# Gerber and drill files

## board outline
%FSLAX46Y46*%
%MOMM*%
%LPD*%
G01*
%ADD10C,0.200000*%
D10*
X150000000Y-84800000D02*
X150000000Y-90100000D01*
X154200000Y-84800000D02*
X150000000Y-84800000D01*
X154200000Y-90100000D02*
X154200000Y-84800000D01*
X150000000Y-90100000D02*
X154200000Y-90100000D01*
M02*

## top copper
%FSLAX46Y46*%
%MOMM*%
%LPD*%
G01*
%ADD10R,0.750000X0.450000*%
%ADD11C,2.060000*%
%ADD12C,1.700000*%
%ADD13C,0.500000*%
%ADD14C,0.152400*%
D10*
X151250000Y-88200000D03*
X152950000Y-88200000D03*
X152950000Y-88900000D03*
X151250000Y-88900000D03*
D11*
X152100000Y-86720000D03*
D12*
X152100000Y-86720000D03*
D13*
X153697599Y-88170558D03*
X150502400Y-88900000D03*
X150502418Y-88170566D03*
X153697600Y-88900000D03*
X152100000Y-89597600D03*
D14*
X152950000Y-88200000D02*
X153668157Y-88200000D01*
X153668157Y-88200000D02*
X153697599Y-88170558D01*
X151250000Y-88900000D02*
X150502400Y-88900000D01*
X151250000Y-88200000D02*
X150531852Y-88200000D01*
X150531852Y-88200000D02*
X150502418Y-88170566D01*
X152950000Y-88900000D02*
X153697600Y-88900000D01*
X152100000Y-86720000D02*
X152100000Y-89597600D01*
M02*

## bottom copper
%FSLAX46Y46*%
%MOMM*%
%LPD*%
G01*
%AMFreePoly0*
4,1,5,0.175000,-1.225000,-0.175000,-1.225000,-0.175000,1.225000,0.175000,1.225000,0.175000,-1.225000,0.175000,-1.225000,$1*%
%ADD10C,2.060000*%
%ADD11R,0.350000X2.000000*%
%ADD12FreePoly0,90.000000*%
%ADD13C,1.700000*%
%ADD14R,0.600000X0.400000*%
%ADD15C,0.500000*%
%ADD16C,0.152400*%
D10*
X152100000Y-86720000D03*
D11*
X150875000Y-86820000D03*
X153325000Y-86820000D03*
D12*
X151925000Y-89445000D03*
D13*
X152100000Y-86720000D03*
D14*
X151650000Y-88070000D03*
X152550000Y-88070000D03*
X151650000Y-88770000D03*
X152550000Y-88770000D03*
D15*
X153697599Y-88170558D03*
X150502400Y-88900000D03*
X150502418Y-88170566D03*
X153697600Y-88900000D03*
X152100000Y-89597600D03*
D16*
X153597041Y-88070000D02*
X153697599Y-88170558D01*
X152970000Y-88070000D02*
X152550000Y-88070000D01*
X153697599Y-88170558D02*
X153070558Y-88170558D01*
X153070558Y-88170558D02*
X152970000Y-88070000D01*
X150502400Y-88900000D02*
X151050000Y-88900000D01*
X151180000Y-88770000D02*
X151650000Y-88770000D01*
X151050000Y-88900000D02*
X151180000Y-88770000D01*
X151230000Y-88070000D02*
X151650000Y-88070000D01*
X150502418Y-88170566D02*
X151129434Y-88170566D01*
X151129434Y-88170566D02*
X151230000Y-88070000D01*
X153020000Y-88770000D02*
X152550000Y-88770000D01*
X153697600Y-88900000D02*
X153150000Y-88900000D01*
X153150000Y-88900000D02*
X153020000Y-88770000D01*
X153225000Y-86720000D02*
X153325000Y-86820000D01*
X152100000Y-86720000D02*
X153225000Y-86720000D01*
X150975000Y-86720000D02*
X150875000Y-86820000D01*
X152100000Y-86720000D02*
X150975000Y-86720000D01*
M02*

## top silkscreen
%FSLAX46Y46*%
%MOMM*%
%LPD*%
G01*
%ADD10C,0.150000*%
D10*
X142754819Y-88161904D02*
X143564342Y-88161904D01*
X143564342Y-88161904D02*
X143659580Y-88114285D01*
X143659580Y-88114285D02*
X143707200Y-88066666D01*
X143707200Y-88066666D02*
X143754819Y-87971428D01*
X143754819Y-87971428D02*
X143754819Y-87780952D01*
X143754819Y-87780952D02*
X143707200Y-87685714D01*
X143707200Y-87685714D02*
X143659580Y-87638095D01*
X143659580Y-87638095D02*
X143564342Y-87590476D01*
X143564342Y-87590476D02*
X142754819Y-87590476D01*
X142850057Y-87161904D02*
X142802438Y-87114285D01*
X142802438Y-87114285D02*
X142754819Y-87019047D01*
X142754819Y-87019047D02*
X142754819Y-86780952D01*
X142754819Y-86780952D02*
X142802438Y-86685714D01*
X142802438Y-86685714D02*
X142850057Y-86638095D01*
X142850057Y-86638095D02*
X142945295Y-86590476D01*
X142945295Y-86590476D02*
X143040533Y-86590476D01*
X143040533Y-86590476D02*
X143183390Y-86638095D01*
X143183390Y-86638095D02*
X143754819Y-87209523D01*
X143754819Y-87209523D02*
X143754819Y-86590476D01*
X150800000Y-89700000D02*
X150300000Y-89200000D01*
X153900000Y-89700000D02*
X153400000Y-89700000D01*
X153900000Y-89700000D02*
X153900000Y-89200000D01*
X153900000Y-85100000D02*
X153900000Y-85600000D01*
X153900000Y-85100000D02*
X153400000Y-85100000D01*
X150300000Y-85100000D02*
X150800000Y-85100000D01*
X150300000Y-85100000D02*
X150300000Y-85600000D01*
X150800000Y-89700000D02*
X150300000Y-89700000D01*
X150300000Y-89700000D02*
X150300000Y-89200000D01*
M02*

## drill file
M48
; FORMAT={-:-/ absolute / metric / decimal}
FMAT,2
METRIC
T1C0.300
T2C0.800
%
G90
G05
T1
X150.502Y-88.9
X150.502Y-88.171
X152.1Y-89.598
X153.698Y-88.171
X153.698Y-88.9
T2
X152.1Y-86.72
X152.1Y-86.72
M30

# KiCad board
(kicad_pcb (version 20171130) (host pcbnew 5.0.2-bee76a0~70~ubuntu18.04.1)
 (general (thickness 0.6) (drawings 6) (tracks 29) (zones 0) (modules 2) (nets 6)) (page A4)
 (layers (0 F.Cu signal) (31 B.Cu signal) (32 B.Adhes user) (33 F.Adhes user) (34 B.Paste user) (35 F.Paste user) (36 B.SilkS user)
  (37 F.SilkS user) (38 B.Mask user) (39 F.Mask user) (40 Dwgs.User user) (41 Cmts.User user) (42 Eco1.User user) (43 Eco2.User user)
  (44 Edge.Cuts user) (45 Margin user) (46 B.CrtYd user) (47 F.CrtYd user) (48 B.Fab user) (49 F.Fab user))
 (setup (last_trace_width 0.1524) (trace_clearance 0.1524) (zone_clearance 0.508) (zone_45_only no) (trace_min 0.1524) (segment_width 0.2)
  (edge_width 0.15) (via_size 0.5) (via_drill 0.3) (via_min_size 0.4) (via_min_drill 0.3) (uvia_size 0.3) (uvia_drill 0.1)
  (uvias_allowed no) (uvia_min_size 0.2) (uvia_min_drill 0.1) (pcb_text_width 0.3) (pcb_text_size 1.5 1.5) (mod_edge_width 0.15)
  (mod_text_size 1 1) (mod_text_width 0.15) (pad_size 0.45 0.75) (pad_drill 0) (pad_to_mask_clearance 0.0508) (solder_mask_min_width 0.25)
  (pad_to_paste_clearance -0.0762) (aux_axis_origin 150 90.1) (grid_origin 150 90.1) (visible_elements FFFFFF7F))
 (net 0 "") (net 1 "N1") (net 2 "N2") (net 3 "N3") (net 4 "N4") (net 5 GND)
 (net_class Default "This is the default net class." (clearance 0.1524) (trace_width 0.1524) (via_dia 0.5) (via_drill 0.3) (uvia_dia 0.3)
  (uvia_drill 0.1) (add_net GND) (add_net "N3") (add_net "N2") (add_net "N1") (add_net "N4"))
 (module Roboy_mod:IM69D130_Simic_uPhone (layer F.Cu) (at 152.1 87.4 90)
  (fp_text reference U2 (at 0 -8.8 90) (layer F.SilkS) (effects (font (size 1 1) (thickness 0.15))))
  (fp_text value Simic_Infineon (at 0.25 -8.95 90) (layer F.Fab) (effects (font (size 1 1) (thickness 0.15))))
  (fp_line (start -2.3 -1.3) (end -1.8 -1.8) (layer F.SilkS) (width 0.15))
  (fp_line (start -2.3 1.8) (end -2.3 1.3) (layer F.SilkS) (width 0.15))
  (fp_line (start -2.3 1.8) (end -1.8 1.8) (layer F.SilkS) (width 0.15))
  (fp_line (start 2.3 1.8) (end 1.8 1.8) (layer F.SilkS) (width 0.15))
  (fp_line (start 2.3 1.8) (end 2.3 1.3) (layer F.SilkS) (width 0.15))
  (fp_line (start 2.3 -1.8) (end 2.3 -1.3) (layer F.SilkS) (width 0.15))
  (fp_line (start 2.3 -1.8) (end 1.8 -1.8) (layer F.SilkS) (width 0.15))
  (fp_line (start -2.3 -1.3) (end -2.3 -1.8) (layer F.SilkS) (width 0.15))
  (fp_line (start -2.3 -1.8) (end -1.8 -1.8) (layer F.SilkS) (width 0.15))
  (pad 2 smd rect (at -0.8 -0.85 90) (size 0.45 0.75) (layers F.Cu F.Paste F.Mask) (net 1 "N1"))
  (pad 4 smd rect (at -0.8 0.85 90) (size 0.45 0.75) (layers F.Cu F.Paste F.Mask) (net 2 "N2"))
  (pad 3 smd rect (at -1.5 0.85 90) (size 0.45 0.75) (layers F.Cu F.Paste F.Mask) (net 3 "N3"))
  (pad 1 smd rect (at -1.5 -0.85 90) (size 0.45 0.75) (layers F.Cu F.Paste F.Mask) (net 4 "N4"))
  (pad 5 thru_hole circle (at 0.68 0 90) (size 2.06 2.06) (drill 0.8) (layers F.Cu) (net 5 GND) (zone_connect 0)))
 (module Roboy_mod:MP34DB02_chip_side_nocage (layer B.Cu) (at 152.1 87.72 90)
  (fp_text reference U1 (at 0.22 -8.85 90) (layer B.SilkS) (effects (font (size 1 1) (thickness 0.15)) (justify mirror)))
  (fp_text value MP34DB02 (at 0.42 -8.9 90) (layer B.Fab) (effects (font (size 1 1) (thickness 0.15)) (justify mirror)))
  (pad 5 smd rect (at 0.9 -1.225 90) (size 2 0.35) (layers B.Cu B.Paste B.Mask) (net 5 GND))
  (pad 5 smd rect (at 0.9 1.225 90) (size 2 0.35) (layers B.Cu B.Paste B.Mask) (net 5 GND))
  (pad 5 smd custom (at -1.725 -0.175 90) (size 0.35 2.45) (layers B.Cu B.Paste B.Mask) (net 5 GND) (zone_connect 0)
   (options (clearance outline) (anchor rect)) (primitives))
  (pad 5 thru_hole circle (at 1 0 90) (size 1.7 1.7) (drill 0.8) (layers B.Cu) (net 5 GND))
  (pad 3 smd rect (at -0.35 -0.45 90) (size 0.4 0.6) (layers B.Cu B.Paste B.Mask) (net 1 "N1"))
  (pad 2 smd rect (at -0.35 0.45 90) (size 0.4 0.6) (layers B.Cu B.Paste B.Mask) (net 2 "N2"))
  (pad 4 smd rect (at -1.05 -0.45 90) (size 0.4 0.6) (layers B.Cu B.Paste B.Mask) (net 4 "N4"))
  (pad 1 smd rect (at -1.05 0.45 90) (size 0.4 0.6) (layers B.Cu B.Paste B.Mask) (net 3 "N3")))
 (gr_line (start 150 84.8) (end 150 90.1) (layer Edge.Cuts) (width 0.2))
 (gr_line (start 154.2 84.8) (end 150 84.8) (layer Edge.Cuts) (width 0.2))
 (gr_line (start 154.2 90.1) (end 154.2 84.8) (layer Edge.Cuts) (width 0.2))
 (gr_line (start 150 90.1) (end 154.2 90.1) (layer Edge.Cuts) (width 0.2))
 (via (at 153.697599 88.170558) (size 0.5) (drill 0.3) (layers F.Cu B.Cu) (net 2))
 (segment (start 152.95 88.2) (end 153.668157 88.2) (width 0.1524) (layer F.Cu) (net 2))
 (segment (start 153.668157 88.2) (end 153.697599 88.170558) (width 0.1524) (layer F.Cu) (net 2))
 (segment (start 153.597041 88.07) (end 153.697599 88.170558) (width 0.1524) (layer B.Cu) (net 2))
 (segment (start 152.97 88.07) (end 152.55 88.07) (width 0.1524) (layer B.Cu) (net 2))
 (segment (start 153.697599 88.170558) (end 153.070558 88.170558) (width 0.1524) (layer B.Cu) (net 2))
 (segment (start 153.070558 88.170558) (end 152.97 88.07) (width 0.1524) (layer B.Cu) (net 2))
 (via (at 150.5024 88.9) (size 0.5) (drill 0.3) (layers F.Cu B.Cu) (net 4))
 (segment (start 151.25 88.9) (end 150.5024 88.9) (width 0.1524) (layer F.Cu) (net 4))
 (segment (start 150.5024 88.9) (end 151.05 88.9) (width 0.1524) (layer B.Cu) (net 4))
 (segment (start 151.18 88.77) (end 151.65 88.77) (width 0.1524) (layer B.Cu) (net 4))
 (segment (start 151.05 88.9) (end 151.18 88.77) (width 0.1524) (layer B.Cu) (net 4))
 (via (at 150.502418 88.170566) (size 0.5) (drill 0.3) (layers F.Cu B.Cu) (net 1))
 (segment (start 151.25 88.2) (end 150.531852 88.2) (width 0.1524) (layer F.Cu) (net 1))
 (segment (start 150.531852 88.2) (end 150.502418 88.170566) (width 0.1524) (layer F.Cu) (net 1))
 (segment (start 151.23 88.07) (end 151.65 88.07) (width 0.1524) (layer B.Cu) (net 1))
 (segment (start 150.502418 88.170566) (end 151.129434 88.170566) (width 0.1524) (layer B.Cu) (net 1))
 (segment (start 151.129434 88.170566) (end 151.23 88.07) (width 0.1524) (layer B.Cu) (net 1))
 (via (at 153.6976 88.9) (size 0.5) (drill 0.3) (layers F.Cu B.Cu) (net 3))
 (segment (start 152.95 88.9) (end 153.6976 88.9) (width 0.1524) (layer F.Cu) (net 3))
 (segment (start 153.02 88.77) (end 152.55 88.77) (width 0.1524) (layer B.Cu) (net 3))
 (segment (start 153.6976 88.9) (end 153.15 88.9) (width 0.1524) (layer B.Cu) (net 3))
 (segment (start 153.15 88.9) (end 153.02 88.77) (width 0.1524) (layer B.Cu) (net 3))
 (segment (start 153.225 86.72) (end 153.325 86.82) (width 0.1524) (layer B.Cu) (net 5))
 (segment (start 152.1 86.72) (end 153.225 86.72) (width 0.1524) (layer B.Cu) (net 5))
 (segment (start 150.975 86.72) (end 150.875 86.82) (width 0.1524) (layer B.Cu) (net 5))
 (segment (start 152.1 86.72) (end 150.975 86.72) (width 0.1524) (layer B.Cu) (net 5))
 (via (at 152.1 89.5976) (size 0.5) (drill 0.3) (layers F.Cu B.Cu) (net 5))
 (segment (start 152.1 86.72) (end 152.1 89.5976) (width 0.1524) (layer F.Cu) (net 5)))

